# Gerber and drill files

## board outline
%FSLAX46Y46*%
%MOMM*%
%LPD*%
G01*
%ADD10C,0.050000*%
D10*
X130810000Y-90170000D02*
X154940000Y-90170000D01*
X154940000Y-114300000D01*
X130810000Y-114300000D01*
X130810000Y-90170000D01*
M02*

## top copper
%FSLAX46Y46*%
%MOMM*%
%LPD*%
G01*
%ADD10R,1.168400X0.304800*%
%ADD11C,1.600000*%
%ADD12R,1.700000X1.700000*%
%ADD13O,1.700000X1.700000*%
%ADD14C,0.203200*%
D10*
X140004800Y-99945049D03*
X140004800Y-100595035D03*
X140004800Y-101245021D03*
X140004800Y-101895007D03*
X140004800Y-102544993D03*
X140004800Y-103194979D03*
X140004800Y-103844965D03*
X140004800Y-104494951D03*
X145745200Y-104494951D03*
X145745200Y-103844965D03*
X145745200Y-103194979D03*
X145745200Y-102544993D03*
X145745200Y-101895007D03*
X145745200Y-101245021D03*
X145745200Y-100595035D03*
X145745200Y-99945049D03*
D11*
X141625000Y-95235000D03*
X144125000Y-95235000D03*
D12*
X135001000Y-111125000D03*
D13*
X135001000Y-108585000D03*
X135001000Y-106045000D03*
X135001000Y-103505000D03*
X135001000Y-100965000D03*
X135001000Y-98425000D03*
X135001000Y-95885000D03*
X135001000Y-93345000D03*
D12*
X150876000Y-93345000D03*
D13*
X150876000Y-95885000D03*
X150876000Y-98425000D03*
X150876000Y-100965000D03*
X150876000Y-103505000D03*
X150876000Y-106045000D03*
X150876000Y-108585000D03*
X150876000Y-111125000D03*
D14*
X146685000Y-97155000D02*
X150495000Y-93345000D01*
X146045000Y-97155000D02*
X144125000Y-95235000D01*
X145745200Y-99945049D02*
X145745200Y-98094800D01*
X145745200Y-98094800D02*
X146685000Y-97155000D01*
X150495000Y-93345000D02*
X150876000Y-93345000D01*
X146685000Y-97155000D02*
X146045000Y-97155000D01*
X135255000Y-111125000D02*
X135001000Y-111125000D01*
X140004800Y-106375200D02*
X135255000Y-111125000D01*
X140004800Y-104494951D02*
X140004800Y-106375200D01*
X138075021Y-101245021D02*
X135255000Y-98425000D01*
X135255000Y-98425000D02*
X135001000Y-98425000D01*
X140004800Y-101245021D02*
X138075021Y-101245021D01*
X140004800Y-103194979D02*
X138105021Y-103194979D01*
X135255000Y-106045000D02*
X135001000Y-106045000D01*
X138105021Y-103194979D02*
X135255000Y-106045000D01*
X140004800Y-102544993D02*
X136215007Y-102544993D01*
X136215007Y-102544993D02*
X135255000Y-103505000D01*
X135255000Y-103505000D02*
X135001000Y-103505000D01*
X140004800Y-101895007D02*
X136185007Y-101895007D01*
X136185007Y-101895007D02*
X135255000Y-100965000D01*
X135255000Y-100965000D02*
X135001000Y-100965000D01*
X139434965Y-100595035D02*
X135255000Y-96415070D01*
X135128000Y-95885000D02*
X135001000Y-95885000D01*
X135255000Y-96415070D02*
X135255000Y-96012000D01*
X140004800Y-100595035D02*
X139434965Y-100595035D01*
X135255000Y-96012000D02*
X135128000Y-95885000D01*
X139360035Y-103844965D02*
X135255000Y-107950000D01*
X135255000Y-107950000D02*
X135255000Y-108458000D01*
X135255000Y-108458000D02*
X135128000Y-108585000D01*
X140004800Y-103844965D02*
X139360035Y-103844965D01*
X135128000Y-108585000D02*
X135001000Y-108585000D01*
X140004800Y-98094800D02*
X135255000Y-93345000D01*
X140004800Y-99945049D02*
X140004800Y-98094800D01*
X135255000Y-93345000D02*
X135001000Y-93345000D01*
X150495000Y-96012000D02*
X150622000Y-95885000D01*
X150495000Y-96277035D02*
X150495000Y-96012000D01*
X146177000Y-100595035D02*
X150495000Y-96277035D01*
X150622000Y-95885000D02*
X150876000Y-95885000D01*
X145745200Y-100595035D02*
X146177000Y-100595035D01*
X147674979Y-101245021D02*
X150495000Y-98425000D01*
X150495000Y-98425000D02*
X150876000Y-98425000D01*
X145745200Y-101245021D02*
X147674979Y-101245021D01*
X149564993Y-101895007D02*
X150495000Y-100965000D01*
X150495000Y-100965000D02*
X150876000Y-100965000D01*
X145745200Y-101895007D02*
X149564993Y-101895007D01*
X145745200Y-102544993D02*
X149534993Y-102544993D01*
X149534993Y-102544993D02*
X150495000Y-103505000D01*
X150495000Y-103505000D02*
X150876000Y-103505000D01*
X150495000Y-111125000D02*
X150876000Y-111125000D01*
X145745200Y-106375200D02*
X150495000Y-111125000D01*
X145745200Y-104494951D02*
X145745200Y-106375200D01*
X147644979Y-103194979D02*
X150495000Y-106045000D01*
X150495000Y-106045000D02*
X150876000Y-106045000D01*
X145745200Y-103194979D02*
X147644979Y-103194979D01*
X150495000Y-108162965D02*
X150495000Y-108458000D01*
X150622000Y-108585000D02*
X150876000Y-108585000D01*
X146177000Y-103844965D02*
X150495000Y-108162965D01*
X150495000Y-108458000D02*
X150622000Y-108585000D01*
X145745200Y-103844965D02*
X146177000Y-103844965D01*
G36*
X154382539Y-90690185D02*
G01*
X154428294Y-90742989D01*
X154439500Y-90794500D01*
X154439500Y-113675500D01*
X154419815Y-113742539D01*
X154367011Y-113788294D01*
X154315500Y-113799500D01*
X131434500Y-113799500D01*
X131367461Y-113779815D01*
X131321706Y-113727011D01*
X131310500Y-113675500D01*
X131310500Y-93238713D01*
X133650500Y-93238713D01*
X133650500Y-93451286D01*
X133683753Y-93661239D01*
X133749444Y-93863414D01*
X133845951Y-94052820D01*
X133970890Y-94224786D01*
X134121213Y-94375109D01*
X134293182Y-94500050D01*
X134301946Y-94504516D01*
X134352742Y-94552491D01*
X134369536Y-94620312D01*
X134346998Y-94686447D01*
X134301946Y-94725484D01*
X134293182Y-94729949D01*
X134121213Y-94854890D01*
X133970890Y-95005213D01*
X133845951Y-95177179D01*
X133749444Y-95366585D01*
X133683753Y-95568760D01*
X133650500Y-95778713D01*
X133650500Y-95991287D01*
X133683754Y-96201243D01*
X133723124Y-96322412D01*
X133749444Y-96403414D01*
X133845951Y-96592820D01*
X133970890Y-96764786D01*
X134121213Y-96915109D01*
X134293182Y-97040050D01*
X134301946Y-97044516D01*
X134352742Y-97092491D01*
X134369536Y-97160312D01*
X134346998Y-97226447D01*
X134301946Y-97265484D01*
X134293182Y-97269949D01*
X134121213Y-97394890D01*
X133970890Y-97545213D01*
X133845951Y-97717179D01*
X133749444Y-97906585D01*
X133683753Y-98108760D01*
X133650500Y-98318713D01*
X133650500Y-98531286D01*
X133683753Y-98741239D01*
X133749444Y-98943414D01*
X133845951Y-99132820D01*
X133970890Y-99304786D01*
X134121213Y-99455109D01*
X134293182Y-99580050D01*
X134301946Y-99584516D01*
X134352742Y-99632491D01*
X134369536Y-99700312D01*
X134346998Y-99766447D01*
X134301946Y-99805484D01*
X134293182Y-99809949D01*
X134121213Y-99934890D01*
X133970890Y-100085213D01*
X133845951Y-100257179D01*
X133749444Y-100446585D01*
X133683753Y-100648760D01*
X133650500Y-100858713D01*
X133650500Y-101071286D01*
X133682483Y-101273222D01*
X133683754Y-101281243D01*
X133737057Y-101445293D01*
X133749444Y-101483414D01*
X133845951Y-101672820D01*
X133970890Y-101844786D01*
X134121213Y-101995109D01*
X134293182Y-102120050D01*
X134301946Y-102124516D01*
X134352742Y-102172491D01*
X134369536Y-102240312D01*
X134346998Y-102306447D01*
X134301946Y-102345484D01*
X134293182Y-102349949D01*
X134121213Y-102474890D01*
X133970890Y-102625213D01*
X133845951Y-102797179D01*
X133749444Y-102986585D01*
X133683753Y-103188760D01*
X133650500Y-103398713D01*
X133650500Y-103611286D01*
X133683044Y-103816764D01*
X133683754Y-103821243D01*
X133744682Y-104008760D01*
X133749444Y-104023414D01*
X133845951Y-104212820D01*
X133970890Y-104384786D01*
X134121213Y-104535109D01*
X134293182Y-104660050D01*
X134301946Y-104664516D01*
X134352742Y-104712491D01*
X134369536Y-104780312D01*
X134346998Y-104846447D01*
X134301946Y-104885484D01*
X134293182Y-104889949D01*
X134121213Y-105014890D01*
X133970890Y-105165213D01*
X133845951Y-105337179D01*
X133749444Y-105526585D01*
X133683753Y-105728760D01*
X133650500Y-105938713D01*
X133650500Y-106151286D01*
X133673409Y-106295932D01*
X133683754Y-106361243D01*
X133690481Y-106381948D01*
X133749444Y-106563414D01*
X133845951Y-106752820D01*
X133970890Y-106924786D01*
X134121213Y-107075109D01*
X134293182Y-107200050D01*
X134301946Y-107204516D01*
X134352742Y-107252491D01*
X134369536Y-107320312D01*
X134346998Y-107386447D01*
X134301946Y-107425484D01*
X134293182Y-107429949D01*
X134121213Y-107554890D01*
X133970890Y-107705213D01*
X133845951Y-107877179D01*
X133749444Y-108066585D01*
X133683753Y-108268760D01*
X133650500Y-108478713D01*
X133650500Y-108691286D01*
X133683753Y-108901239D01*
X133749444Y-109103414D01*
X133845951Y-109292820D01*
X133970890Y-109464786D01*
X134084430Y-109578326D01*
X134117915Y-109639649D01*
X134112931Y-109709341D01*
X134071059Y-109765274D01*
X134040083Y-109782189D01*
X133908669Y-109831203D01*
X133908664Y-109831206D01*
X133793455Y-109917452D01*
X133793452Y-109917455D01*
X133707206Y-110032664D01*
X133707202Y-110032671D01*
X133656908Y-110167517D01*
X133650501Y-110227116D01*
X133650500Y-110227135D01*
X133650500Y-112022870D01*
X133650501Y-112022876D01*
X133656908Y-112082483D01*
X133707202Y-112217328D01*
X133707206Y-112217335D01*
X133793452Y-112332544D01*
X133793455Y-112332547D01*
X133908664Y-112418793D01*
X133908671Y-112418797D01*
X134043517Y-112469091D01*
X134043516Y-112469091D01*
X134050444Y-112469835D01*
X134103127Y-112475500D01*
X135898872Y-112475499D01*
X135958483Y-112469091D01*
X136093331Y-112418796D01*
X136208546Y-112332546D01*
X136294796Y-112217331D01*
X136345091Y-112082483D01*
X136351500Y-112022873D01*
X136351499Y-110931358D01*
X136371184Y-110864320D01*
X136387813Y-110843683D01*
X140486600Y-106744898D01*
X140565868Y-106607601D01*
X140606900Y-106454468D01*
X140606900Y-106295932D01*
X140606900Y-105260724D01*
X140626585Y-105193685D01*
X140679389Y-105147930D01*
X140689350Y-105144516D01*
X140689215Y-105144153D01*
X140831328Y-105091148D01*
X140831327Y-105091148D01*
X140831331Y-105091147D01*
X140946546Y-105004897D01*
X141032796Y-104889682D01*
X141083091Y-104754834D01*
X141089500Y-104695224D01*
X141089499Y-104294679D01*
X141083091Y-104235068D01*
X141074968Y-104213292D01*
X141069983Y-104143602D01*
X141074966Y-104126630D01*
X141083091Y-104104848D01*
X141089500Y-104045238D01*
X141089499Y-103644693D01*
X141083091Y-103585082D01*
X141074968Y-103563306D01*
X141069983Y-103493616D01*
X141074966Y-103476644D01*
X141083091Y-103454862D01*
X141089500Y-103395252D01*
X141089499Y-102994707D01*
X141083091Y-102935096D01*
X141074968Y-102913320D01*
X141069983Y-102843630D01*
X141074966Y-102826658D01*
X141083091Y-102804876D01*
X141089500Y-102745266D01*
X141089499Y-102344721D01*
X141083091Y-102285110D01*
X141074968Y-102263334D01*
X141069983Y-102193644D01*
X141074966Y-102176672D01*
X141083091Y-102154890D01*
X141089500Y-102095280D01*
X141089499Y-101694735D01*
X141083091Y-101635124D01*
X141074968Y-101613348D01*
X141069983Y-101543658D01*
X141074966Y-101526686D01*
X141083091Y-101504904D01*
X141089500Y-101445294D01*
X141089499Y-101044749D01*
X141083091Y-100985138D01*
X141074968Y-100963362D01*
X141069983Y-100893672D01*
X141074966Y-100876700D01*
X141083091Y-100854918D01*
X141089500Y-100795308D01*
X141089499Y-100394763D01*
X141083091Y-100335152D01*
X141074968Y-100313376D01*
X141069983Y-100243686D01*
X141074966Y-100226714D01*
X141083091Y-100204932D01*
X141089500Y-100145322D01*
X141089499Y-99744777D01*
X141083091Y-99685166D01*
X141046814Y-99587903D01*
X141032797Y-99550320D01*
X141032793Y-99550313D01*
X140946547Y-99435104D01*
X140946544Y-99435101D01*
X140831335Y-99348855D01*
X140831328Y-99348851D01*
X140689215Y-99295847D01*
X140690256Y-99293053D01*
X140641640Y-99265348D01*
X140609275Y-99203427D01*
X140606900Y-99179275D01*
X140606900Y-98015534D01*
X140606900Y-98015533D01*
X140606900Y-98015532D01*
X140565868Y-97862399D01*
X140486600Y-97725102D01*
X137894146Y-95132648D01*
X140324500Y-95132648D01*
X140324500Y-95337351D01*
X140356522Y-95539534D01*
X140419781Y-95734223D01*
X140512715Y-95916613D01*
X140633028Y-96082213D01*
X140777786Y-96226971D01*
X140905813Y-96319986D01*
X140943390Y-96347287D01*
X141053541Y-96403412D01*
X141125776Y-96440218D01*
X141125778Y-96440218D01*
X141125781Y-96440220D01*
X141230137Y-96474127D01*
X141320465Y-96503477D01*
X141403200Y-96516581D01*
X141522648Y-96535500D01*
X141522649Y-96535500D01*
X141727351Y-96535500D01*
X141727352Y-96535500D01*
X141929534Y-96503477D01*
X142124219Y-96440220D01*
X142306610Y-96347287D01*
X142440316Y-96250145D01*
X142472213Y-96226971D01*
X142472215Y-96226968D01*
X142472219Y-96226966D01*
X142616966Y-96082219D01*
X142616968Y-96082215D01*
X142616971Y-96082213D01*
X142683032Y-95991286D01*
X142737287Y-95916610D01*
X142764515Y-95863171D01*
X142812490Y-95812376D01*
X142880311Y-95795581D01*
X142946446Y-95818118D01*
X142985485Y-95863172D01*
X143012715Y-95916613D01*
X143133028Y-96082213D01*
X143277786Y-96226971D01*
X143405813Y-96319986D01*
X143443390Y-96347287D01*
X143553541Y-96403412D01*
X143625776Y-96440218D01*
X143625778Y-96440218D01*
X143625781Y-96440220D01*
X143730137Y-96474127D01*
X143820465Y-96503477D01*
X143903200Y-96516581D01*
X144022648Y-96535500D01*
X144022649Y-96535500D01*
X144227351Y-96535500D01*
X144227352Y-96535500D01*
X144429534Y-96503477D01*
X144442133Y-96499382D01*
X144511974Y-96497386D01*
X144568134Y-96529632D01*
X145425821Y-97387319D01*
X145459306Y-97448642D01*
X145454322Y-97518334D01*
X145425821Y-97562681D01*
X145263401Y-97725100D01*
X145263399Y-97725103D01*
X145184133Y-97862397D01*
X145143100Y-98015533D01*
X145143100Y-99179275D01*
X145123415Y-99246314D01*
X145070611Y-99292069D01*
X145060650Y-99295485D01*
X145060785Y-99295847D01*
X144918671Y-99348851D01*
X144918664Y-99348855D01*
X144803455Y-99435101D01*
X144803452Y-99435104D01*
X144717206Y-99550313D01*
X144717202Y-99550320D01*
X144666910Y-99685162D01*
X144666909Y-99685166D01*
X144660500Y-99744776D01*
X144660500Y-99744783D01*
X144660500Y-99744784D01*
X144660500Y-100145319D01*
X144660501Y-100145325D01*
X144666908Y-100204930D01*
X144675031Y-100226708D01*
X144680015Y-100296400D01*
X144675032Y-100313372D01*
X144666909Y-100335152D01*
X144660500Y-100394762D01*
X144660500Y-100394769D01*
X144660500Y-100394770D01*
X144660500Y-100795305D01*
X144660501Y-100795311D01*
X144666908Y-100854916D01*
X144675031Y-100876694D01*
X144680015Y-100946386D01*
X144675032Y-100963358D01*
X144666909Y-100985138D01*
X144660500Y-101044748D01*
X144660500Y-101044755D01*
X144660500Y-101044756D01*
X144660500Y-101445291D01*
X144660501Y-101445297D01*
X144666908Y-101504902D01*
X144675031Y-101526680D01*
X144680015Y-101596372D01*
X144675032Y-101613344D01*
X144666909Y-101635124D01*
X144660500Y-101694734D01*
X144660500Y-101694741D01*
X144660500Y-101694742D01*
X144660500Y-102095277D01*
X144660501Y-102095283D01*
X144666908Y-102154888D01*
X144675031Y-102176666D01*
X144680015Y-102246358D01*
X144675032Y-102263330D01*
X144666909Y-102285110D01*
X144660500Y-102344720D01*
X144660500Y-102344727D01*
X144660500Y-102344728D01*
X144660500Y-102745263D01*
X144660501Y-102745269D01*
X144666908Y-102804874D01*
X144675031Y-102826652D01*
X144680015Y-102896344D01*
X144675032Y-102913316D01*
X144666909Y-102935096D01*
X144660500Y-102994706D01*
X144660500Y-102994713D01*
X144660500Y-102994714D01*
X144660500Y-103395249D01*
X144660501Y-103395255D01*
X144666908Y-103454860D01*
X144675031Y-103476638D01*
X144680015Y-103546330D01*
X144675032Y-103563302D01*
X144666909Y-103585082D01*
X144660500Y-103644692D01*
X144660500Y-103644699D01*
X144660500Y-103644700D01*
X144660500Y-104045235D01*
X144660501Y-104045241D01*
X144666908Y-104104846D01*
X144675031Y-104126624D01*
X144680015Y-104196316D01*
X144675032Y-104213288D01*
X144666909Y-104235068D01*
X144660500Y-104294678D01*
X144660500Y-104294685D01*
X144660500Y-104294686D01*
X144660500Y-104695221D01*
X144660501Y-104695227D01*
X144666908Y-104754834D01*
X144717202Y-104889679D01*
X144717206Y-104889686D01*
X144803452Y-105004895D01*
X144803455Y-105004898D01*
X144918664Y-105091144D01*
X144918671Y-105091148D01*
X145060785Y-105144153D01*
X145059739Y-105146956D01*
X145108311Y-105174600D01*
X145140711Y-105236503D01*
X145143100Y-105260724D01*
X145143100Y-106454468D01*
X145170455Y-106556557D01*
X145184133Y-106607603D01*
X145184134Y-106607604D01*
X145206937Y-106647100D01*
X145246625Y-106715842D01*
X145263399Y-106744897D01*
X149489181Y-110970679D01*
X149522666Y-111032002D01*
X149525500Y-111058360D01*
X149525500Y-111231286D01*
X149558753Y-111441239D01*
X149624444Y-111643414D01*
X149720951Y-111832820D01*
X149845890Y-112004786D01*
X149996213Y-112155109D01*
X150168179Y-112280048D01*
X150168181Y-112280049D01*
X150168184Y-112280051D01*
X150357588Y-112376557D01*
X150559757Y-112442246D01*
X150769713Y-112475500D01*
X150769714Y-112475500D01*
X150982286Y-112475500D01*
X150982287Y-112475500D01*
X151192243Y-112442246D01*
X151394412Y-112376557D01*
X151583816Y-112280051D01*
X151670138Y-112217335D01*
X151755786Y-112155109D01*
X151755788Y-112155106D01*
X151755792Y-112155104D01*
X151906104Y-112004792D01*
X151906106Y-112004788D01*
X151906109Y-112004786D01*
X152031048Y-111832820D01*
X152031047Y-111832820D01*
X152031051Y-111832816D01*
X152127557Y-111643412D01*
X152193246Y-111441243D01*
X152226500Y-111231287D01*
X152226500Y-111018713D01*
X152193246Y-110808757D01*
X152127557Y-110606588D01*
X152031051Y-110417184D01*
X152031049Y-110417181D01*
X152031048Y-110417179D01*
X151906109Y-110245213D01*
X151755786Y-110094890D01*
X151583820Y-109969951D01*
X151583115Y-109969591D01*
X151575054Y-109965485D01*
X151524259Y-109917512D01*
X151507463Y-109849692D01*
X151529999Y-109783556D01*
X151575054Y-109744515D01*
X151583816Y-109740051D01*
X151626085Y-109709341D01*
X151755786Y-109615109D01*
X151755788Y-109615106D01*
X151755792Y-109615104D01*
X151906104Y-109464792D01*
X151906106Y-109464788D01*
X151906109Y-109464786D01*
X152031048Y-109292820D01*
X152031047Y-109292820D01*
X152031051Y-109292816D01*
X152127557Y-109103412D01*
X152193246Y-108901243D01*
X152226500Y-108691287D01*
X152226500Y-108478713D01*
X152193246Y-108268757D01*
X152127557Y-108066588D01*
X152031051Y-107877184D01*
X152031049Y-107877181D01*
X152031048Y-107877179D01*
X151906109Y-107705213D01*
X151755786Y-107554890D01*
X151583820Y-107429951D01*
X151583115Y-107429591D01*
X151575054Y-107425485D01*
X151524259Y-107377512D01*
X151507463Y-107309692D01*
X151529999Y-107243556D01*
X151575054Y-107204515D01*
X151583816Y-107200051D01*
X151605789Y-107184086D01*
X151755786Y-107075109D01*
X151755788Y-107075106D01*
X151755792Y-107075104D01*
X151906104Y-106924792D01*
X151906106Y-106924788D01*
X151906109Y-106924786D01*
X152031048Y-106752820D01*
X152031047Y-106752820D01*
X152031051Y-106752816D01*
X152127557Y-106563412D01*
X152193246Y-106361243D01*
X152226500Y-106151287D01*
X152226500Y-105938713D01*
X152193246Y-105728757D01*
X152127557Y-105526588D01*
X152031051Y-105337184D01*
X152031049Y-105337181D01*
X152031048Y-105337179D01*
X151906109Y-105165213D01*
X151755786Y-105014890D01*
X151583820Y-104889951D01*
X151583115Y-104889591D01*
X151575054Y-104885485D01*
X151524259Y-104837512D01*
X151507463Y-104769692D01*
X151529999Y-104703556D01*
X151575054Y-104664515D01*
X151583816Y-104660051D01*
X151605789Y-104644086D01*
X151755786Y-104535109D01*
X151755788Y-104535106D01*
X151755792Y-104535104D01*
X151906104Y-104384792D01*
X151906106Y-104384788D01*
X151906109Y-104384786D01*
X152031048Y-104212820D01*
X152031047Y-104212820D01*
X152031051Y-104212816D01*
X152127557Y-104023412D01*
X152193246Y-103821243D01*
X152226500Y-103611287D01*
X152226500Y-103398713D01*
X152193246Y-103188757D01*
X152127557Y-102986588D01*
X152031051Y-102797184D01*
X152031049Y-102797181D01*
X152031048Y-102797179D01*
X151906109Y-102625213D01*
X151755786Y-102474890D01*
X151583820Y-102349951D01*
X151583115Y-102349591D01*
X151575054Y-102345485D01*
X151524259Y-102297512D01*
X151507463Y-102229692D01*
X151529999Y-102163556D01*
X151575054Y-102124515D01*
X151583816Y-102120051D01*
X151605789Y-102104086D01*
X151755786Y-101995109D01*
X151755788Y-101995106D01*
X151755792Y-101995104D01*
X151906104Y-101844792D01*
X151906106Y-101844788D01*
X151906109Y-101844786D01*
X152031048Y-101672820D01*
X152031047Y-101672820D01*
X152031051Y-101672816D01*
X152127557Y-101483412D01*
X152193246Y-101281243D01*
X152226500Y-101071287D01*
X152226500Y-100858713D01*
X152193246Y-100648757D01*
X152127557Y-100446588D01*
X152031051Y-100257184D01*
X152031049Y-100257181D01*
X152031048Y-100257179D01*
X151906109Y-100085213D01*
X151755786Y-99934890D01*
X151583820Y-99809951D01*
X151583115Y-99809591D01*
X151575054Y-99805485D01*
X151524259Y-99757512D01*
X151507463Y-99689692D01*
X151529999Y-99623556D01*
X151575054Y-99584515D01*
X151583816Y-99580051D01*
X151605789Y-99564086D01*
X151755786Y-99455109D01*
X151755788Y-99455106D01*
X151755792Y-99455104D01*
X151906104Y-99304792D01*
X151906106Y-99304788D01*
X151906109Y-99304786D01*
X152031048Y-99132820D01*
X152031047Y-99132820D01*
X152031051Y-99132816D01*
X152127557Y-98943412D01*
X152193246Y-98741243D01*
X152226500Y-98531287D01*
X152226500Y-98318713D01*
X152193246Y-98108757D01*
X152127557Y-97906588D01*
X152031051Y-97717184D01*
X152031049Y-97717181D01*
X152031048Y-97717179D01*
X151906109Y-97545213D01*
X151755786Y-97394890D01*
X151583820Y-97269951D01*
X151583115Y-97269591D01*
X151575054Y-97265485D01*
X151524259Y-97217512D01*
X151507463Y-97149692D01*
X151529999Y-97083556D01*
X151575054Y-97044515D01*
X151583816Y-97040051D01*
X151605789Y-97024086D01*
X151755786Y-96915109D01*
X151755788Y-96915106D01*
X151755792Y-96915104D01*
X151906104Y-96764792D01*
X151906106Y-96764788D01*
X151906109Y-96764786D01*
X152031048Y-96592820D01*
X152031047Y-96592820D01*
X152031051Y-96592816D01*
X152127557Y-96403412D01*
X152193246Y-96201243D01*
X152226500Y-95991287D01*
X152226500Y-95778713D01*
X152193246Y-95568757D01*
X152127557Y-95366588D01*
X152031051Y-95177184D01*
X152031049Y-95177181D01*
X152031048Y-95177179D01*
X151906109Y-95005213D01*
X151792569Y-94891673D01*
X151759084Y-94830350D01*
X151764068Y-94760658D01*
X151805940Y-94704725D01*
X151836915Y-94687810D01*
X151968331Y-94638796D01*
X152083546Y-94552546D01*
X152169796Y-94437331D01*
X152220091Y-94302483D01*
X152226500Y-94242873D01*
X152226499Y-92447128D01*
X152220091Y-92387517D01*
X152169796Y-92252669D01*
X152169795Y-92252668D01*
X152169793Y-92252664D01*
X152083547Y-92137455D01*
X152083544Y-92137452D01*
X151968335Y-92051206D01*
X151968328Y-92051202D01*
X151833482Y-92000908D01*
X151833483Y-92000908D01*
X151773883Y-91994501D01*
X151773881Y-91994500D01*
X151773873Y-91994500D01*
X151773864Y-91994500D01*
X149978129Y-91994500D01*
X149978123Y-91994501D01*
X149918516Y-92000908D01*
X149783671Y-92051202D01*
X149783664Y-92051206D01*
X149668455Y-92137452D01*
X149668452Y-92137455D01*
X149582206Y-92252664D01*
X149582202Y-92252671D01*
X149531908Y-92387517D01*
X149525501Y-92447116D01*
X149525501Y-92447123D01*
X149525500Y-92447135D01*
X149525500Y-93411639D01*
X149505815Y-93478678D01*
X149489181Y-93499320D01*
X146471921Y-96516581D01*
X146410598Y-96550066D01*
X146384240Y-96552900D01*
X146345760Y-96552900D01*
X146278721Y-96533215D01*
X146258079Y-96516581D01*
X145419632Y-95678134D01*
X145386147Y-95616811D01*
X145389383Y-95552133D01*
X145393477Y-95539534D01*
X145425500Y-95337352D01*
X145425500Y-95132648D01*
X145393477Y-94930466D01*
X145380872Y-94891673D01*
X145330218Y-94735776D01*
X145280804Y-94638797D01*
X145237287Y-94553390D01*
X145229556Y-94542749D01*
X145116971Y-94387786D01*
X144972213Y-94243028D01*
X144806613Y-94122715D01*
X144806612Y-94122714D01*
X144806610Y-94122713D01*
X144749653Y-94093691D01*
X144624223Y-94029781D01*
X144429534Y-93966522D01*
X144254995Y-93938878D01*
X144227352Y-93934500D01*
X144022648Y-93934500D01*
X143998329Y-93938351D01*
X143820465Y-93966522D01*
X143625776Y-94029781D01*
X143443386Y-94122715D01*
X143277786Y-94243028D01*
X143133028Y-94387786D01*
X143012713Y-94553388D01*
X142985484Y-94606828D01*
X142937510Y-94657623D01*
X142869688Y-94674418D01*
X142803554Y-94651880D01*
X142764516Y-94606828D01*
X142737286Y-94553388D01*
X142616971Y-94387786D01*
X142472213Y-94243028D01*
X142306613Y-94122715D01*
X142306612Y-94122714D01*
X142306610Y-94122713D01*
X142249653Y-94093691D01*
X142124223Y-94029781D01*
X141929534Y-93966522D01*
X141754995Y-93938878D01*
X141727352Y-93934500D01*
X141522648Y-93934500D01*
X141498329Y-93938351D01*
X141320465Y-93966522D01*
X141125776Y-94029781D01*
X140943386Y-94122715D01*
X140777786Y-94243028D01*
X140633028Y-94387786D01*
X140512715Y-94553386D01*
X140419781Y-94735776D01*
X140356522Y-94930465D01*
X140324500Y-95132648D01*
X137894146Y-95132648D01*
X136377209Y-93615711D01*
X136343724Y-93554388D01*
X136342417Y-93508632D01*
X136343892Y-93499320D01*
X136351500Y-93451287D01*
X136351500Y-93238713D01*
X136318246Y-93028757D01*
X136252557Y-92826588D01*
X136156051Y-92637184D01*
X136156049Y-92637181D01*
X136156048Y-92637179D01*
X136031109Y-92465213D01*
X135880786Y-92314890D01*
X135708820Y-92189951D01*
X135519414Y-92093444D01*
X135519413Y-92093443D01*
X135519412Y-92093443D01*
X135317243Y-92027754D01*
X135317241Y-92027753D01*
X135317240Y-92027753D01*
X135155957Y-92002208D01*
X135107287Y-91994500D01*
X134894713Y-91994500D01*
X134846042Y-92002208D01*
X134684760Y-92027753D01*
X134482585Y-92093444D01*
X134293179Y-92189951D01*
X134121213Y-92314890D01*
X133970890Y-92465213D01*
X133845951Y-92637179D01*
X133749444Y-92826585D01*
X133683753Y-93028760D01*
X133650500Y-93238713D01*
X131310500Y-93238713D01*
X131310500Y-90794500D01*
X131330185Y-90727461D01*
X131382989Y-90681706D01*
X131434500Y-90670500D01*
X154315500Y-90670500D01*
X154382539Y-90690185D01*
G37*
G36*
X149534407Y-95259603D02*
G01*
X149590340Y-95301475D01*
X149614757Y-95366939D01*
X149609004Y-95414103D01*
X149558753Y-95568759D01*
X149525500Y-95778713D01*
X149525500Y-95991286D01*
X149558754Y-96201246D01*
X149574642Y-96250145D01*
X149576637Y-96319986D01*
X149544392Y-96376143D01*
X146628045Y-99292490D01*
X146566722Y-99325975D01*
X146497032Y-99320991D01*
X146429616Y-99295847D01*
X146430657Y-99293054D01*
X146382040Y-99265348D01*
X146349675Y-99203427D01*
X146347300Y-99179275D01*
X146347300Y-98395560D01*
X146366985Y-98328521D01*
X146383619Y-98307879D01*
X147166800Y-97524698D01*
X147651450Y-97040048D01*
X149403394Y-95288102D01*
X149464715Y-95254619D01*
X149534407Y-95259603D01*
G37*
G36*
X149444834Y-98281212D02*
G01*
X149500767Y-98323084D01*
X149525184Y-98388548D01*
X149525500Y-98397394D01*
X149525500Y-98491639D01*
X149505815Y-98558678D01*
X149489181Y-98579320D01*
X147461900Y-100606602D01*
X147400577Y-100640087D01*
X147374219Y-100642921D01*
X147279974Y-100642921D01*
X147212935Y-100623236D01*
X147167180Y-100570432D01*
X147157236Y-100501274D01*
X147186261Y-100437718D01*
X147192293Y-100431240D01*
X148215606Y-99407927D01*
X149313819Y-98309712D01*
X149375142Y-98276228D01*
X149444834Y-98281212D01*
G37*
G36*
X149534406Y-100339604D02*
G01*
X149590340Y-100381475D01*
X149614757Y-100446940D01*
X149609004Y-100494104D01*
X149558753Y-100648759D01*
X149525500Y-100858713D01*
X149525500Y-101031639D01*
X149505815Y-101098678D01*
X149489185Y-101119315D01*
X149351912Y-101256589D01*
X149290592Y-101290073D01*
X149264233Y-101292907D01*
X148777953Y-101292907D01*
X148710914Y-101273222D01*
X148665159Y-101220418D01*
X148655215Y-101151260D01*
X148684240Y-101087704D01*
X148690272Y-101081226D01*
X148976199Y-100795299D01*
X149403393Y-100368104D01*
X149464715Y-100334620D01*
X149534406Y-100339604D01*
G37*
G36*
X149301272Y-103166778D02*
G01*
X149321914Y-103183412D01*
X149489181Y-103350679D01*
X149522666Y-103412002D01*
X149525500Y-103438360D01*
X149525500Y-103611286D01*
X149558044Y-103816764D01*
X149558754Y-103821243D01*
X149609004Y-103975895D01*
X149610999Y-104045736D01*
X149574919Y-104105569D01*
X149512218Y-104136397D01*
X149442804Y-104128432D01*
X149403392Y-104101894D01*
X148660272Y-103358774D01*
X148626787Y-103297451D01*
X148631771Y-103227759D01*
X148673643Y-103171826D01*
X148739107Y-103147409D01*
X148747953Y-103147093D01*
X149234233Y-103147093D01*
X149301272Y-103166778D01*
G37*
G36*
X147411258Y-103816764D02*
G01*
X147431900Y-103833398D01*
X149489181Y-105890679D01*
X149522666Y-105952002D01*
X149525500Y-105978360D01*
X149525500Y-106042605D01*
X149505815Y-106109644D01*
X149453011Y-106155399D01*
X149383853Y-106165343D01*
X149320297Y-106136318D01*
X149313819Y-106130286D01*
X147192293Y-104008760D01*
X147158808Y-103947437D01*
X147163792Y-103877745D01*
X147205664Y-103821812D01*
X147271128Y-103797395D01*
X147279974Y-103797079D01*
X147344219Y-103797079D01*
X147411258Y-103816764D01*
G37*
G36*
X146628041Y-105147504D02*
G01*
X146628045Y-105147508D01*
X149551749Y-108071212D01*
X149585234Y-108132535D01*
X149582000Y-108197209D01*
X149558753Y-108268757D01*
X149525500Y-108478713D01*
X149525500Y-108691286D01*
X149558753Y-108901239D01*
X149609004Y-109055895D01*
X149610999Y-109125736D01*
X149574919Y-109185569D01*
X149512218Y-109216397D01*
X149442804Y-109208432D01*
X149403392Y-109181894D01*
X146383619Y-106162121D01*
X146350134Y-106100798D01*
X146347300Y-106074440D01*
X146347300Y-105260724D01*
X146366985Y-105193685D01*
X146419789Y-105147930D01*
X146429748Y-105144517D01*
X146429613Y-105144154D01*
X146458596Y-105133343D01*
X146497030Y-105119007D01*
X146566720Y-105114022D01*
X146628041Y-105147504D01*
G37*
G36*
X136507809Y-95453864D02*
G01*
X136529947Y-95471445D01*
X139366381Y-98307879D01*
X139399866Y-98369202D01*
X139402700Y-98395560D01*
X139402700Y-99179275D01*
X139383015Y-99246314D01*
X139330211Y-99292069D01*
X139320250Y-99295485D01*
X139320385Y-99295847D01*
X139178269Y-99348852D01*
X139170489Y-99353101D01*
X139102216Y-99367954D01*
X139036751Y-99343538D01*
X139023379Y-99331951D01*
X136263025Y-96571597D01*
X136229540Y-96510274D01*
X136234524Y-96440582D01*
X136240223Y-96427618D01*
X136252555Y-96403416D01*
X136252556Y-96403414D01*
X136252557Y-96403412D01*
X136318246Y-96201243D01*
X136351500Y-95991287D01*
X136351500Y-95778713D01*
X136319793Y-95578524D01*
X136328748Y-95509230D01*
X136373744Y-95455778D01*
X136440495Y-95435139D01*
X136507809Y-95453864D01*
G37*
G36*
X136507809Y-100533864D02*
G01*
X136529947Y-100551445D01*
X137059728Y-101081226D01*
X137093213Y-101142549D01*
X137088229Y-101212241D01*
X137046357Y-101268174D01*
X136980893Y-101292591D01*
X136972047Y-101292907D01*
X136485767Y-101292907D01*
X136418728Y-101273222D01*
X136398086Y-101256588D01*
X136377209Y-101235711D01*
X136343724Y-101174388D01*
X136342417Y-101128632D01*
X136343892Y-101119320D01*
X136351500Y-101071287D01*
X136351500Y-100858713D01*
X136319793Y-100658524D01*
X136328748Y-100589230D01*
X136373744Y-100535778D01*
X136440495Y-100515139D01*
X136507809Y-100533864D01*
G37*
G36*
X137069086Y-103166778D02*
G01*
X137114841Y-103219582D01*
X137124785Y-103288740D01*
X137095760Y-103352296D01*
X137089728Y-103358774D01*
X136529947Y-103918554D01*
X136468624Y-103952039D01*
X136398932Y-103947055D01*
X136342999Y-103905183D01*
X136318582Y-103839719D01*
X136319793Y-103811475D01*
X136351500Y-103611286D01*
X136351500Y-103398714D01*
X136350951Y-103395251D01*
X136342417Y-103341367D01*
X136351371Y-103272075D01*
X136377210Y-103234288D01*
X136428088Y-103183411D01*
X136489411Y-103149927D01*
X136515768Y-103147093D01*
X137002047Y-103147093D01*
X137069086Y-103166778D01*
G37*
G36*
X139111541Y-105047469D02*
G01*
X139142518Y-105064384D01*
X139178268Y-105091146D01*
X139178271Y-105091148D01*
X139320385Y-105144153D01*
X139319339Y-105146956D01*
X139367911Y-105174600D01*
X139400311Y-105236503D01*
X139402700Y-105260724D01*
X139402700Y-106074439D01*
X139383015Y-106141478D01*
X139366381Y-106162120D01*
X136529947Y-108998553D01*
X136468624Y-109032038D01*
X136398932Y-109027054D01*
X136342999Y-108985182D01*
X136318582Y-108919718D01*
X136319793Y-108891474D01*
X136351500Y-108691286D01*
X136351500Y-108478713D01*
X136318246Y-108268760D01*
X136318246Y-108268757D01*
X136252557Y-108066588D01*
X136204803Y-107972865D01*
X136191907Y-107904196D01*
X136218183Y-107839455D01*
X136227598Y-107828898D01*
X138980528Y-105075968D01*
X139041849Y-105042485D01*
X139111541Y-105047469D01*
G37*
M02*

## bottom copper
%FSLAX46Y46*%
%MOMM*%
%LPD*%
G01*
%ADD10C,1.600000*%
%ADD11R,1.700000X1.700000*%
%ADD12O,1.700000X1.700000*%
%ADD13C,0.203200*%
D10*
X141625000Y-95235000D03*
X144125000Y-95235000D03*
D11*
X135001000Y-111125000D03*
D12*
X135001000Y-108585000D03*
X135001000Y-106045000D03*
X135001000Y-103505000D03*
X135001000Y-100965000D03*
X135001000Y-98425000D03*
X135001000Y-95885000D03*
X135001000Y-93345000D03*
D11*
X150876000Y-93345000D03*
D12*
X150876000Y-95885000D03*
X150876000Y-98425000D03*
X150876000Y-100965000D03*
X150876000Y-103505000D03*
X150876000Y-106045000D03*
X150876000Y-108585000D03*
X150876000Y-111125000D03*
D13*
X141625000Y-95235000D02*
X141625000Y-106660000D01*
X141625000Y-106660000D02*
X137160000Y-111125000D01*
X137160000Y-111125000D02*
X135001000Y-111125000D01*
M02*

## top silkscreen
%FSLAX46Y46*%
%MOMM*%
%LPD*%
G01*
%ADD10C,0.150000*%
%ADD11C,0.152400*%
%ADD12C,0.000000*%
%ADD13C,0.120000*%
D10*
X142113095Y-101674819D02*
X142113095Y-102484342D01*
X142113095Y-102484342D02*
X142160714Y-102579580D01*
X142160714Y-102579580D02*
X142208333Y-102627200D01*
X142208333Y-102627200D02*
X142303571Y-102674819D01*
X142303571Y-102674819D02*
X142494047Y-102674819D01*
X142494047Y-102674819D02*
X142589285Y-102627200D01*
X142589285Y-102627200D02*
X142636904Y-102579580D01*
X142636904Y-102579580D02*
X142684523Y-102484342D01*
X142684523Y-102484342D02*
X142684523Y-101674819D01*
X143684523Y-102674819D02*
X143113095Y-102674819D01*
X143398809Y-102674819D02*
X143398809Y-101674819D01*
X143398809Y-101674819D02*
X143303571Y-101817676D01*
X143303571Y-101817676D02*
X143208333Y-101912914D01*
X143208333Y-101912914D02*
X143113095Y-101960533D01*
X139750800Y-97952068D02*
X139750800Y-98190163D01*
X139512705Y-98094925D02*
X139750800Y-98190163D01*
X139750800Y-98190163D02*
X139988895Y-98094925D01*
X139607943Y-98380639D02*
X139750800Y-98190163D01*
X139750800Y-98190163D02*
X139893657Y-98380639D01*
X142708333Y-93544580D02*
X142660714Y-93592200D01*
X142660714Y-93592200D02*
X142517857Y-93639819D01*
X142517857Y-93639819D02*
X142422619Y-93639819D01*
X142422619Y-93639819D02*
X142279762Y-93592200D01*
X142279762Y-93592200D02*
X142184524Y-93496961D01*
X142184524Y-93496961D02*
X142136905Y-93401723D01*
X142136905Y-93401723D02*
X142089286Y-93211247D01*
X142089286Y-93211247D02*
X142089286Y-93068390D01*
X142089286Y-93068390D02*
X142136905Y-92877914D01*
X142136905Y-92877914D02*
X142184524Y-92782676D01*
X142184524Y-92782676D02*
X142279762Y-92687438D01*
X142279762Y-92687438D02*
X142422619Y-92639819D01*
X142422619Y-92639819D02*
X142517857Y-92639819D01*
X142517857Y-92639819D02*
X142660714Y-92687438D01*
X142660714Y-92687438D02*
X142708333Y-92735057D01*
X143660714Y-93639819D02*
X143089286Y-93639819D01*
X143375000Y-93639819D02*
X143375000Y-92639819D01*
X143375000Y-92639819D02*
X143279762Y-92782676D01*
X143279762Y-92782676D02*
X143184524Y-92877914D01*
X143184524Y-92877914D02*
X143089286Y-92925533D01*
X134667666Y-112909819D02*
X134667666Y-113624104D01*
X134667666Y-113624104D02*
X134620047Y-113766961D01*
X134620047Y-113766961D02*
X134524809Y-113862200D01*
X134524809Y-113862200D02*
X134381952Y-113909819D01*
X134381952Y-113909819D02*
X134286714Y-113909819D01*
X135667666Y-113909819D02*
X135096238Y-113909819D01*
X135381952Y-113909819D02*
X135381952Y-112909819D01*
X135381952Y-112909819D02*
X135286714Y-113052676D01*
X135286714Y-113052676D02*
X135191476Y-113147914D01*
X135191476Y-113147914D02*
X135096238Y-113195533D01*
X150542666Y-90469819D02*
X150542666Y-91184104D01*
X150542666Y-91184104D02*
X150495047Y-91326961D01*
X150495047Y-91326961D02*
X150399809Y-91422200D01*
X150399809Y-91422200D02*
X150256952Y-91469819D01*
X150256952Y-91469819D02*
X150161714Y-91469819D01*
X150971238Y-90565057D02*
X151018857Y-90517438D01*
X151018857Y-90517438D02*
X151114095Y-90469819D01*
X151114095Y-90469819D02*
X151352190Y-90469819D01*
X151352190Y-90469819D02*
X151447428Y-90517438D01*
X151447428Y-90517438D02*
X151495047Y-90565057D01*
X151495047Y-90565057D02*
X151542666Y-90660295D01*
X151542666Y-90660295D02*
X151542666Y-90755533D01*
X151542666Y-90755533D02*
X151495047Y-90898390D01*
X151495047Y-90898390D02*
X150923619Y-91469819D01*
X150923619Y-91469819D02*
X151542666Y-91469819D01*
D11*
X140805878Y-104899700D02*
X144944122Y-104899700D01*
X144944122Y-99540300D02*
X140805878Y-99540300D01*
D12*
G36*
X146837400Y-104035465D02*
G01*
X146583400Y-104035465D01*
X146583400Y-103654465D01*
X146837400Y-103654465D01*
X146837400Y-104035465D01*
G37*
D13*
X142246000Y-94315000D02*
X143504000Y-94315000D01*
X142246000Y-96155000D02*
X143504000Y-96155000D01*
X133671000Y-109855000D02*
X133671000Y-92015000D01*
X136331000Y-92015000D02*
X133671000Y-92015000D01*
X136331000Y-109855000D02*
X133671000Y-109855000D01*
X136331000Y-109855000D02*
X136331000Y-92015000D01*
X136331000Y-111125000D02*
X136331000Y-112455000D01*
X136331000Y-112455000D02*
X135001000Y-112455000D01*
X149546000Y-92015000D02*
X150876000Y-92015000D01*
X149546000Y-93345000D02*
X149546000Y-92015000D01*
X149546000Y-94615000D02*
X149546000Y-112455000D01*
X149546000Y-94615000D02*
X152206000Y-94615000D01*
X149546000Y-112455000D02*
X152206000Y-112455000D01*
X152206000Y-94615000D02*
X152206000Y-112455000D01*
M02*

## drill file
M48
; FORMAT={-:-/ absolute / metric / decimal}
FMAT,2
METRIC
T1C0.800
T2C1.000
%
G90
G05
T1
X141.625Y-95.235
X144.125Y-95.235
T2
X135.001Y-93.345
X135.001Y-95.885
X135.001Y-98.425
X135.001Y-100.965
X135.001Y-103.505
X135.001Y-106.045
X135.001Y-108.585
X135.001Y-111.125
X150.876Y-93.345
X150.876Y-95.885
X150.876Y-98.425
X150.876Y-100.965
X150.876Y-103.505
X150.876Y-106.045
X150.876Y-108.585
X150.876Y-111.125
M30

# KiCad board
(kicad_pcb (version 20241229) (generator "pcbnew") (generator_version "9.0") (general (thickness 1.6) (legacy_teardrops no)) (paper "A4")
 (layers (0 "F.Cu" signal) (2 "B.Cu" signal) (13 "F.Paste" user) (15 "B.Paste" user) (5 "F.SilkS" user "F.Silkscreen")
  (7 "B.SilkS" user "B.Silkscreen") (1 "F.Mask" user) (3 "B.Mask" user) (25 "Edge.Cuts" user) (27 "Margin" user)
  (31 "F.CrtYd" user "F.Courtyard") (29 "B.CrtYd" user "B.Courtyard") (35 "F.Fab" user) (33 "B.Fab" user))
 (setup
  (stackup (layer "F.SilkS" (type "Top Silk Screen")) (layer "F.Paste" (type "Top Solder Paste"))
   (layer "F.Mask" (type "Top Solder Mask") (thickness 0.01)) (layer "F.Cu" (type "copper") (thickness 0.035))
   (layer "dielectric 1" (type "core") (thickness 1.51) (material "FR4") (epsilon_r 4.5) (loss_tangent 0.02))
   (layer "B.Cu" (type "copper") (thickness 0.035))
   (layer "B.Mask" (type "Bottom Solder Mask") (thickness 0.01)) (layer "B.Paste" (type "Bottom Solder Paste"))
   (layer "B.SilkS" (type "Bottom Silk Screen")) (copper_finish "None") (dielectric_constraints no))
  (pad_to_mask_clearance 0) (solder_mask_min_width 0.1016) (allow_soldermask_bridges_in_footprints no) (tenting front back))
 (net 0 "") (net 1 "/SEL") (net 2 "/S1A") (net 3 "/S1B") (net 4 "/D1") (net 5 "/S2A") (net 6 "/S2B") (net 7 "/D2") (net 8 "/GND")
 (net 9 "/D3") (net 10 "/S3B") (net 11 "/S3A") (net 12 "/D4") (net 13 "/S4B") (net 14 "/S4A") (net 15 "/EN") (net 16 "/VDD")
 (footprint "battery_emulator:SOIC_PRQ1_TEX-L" (layer "F.Cu") (at 142.875 102.22)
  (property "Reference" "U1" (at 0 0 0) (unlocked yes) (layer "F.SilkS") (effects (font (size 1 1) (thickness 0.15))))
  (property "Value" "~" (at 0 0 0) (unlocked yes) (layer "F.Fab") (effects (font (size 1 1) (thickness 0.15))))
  (fp_line (start -2.069122 2.6797) (end 2.069122 2.6797) (stroke (width 0.1524) (type solid)) (layer "F.SilkS"))
  (fp_line (start 2.069122 -2.6797) (end -2.069122 -2.6797) (stroke (width 0.1524) (type solid)) (layer "F.SilkS"))
  (fp_poly
   (pts (xy 3.9624 1.434465) (xy 3.9624 1.815465) (xy 3.7084 1.815465) (xy 3.7084 1.434465)) (stroke (width 0) (type solid)) (fill yes)
   (layer "F.SilkS"))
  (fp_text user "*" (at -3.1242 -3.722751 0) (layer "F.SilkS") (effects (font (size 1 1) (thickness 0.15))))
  (pad "1" smd rect (at -2.8702 -2.274951) (size 1.1684 0.3048) (layers "F.Cu" "F.Mask" "F.Paste") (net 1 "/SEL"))
  (pad "2" smd rect (at -2.8702 -1.624965) (size 1.1684 0.3048) (layers "F.Cu" "F.Mask" "F.Paste") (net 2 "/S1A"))
  (pad "3" smd rect (at -2.8702 -0.974979) (size 1.1684 0.3048) (layers "F.Cu" "F.Mask" "F.Paste") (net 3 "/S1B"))
  (pad "4" smd rect (at -2.8702 -0.324993) (size 1.1684 0.3048) (layers "F.Cu" "F.Mask" "F.Paste") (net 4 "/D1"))
  (pad "5" smd rect (at -2.8702 0.324993) (size 1.1684 0.3048) (layers "F.Cu" "F.Mask" "F.Paste") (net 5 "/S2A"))
  (pad "6" smd rect (at -2.8702 0.974979) (size 1.1684 0.3048) (layers "F.Cu" "F.Mask" "F.Paste") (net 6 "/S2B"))
  (pad "7" smd rect (at -2.8702 1.624965) (size 1.1684 0.3048) (layers "F.Cu" "F.Mask" "F.Paste") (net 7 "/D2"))
  (pad "8" smd rect (at -2.8702 2.274951) (size 1.1684 0.3048) (layers "F.Cu" "F.Mask" "F.Paste") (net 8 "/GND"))
  (pad "9" smd rect (at 2.8702 2.274951) (size 1.1684 0.3048) (layers "F.Cu" "F.Mask" "F.Paste") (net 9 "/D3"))
  (pad "10" smd rect (at 2.8702 1.624965) (size 1.1684 0.3048) (layers "F.Cu" "F.Mask" "F.Paste") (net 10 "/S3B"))
  (pad "11" smd rect (at 2.8702 0.974979) (size 1.1684 0.3048) (layers "F.Cu" "F.Mask" "F.Paste") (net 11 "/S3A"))
  (pad "12" smd rect (at 2.8702 0.324993) (size 1.1684 0.3048) (layers "F.Cu" "F.Mask" "F.Paste") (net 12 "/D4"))
  (pad "13" smd rect (at 2.8702 -0.324993) (size 1.1684 0.3048) (layers "F.Cu" "F.Mask" "F.Paste") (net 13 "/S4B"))
  (pad "14" smd rect (at 2.8702 -0.974979) (size 1.1684 0.3048) (layers "F.Cu" "F.Mask" "F.Paste") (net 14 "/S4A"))
  (pad "15" smd rect (at 2.8702 -1.624965) (size 1.1684 0.3048) (layers "F.Cu" "F.Mask" "F.Paste") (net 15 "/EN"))
  (pad "16" smd rect (at 2.8702 -2.274951) (size 1.1684 0.3048) (layers "F.Cu" "F.Mask" "F.Paste") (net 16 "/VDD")))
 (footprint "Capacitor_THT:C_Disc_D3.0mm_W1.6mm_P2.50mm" (layer "F.Cu") (at 141.625 95.235)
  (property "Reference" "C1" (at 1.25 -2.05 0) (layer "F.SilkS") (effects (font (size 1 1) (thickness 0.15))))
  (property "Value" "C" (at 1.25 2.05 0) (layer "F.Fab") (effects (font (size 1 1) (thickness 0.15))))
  (fp_line (start 0.621 -0.92) (end 1.879 -0.92) (stroke (width 0.12) (type solid)) (layer "F.SilkS"))
  (fp_line (start 0.621 0.92) (end 1.879 0.92) (stroke (width 0.12) (type solid)) (layer "F.SilkS"))
  (pad "1" thru_hole circle (at 0 0) (size 1.6 1.6) (drill 0.8) (layers "*.Cu" "*.Mask") (remove_unused_layers no) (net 8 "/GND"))
  (pad "2" thru_hole circle (at 2.5 0) (size 1.6 1.6) (drill 0.8) (layers "*.Cu" "*.Mask") (remove_unused_layers no) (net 16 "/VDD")))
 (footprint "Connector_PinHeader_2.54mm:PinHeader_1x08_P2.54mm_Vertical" (layer "F.Cu") (at 135.001 111.125 180)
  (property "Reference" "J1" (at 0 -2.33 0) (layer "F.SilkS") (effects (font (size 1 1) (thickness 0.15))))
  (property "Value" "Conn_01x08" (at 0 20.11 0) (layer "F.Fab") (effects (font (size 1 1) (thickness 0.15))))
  (fp_line (start 1.33 1.27) (end 1.33 19.11) (stroke (width 0.12) (type solid)) (layer "F.SilkS"))
  (fp_line (start -1.33 19.11) (end 1.33 19.11) (stroke (width 0.12) (type solid)) (layer "F.SilkS"))
  (fp_line (start -1.33 1.27) (end 1.33 1.27) (stroke (width 0.12) (type solid)) (layer "F.SilkS"))
  (fp_line (start -1.33 1.27) (end -1.33 19.11) (stroke (width 0.12) (type solid)) (layer "F.SilkS"))
  (fp_line (start -1.33 0) (end -1.33 -1.33) (stroke (width 0.12) (type solid)) (layer "F.SilkS"))
  (fp_line (start -1.33 -1.33) (end 0 -1.33) (stroke (width 0.12) (type solid)) (layer "F.SilkS"))
  (pad "1" thru_hole rect (at 0 0 180) (size 1.7 1.7) (drill 1) (layers "*.Cu" "*.Mask") (remove_unused_layers no) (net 8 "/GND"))
  (pad "2" thru_hole oval (at 0 2.54 180) (size 1.7 1.7) (drill 1) (layers "*.Cu" "*.Mask") (remove_unused_layers no) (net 7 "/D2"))
  (pad "3" thru_hole oval (at 0 5.08 180) (size 1.7 1.7) (drill 1) (layers "*.Cu" "*.Mask") (remove_unused_layers no) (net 6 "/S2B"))
  (pad "4" thru_hole oval (at 0 7.62 180) (size 1.7 1.7) (drill 1) (layers "*.Cu" "*.Mask") (remove_unused_layers no) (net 5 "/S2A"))
  (pad "5" thru_hole oval (at 0 10.16 180) (size 1.7 1.7) (drill 1) (layers "*.Cu" "*.Mask") (remove_unused_layers no) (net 4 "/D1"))
  (pad "6" thru_hole oval (at 0 12.7 180) (size 1.7 1.7) (drill 1) (layers "*.Cu" "*.Mask") (remove_unused_layers no) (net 3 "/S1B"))
  (pad "7" thru_hole oval (at 0 15.24 180) (size 1.7 1.7) (drill 1) (layers "*.Cu" "*.Mask") (remove_unused_layers no) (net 2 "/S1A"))
  (pad "8" thru_hole oval (at 0 17.78 180) (size 1.7 1.7) (drill 1) (layers "*.Cu" "*.Mask") (remove_unused_layers no) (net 1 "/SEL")))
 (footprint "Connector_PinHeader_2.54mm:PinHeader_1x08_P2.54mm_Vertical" (layer "F.Cu") (at 150.876 93.345)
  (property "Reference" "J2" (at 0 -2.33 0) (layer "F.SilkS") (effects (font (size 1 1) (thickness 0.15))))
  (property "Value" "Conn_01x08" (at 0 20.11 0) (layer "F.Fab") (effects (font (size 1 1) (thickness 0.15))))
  (fp_line (start -1.33 -1.33) (end 0 -1.33) (stroke (width 0.12) (type solid)) (layer "F.SilkS"))
  (fp_line (start -1.33 0) (end -1.33 -1.33) (stroke (width 0.12) (type solid)) (layer "F.SilkS"))
  (fp_line (start -1.33 1.27) (end -1.33 19.11) (stroke (width 0.12) (type solid)) (layer "F.SilkS"))
  (fp_line (start -1.33 1.27) (end 1.33 1.27) (stroke (width 0.12) (type solid)) (layer "F.SilkS"))
  (fp_line (start -1.33 19.11) (end 1.33 19.11) (stroke (width 0.12) (type solid)) (layer "F.SilkS"))
  (fp_line (start 1.33 1.27) (end 1.33 19.11) (stroke (width 0.12) (type solid)) (layer "F.SilkS"))
  (pad "1" thru_hole rect (at 0 0) (size 1.7 1.7) (drill 1) (layers "*.Cu" "*.Mask") (remove_unused_layers no) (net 16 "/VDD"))
  (pad "2" thru_hole oval (at 0 2.54) (size 1.7 1.7) (drill 1) (layers "*.Cu" "*.Mask") (remove_unused_layers no) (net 15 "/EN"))
  (pad "3" thru_hole oval (at 0 5.08) (size 1.7 1.7) (drill 1) (layers "*.Cu" "*.Mask") (remove_unused_layers no) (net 14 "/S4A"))
  (pad "4" thru_hole oval (at 0 7.62) (size 1.7 1.7) (drill 1) (layers "*.Cu" "*.Mask") (remove_unused_layers no) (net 13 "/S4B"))
  (pad "5" thru_hole oval (at 0 10.16) (size 1.7 1.7) (drill 1) (layers "*.Cu" "*.Mask") (remove_unused_layers no) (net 12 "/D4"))
  (pad "6" thru_hole oval (at 0 12.7) (size 1.7 1.7) (drill 1) (layers "*.Cu" "*.Mask") (remove_unused_layers no) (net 11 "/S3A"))
  (pad "7" thru_hole oval (at 0 15.24) (size 1.7 1.7) (drill 1) (layers "*.Cu" "*.Mask") (remove_unused_layers no) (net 10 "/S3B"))
  (pad "8" thru_hole oval (at 0 17.78) (size 1.7 1.7) (drill 1) (layers "*.Cu" "*.Mask") (remove_unused_layers no) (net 9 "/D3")))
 (gr_rect (start 130.81 90.17) (end 154.94 114.3) (stroke (width 0.05) (type solid)) (fill no) (layer "Edge.Cuts"))
 (segment (start 146.685 97.155) (end 150.495 93.345) (width 0.2032) (layer "F.Cu") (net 16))
 (segment (start 146.045 97.155) (end 144.125 95.235) (width 0.2032) (layer "F.Cu") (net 16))
 (segment (start 145.7452 99.945049) (end 145.7452 98.0948) (width 0.2032) (layer "F.Cu") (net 16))
 (segment (start 145.7452 98.0948) (end 146.685 97.155) (width 0.2032) (layer "F.Cu") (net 16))
 (segment (start 150.495 93.345) (end 150.876 93.345) (width 0.2032) (layer "F.Cu") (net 16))
 (segment (start 146.685 97.155) (end 146.045 97.155) (width 0.2032) (layer "F.Cu") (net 16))
 (segment (start 135.255 111.125) (end 135.001 111.125) (width 0.2032) (layer "F.Cu") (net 8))
 (segment (start 140.0048 106.3752) (end 135.255 111.125) (width 0.2032) (layer "F.Cu") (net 8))
 (segment (start 140.0048 104.494951) (end 140.0048 106.3752) (width 0.2032) (layer "F.Cu") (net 8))
 (segment (start 141.625 95.235) (end 141.625 106.66) (width 0.2032) (layer "B.Cu") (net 8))
 (segment (start 141.625 106.66) (end 137.16 111.125) (width 0.2032) (layer "B.Cu") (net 8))
 (segment (start 137.16 111.125) (end 135.001 111.125) (width 0.2032) (layer "B.Cu") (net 8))
 (segment (start 138.075021 101.245021) (end 135.255 98.425) (width 0.2032) (layer "F.Cu") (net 3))
 (segment (start 135.255 98.425) (end 135.001 98.425) (width 0.2032) (layer "F.Cu") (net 3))
 (segment (start 140.0048 101.245021) (end 138.075021 101.245021) (width 0.2032) (layer "F.Cu") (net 3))
 (segment (start 140.0048 103.194979) (end 138.105021 103.194979) (width 0.2032) (layer "F.Cu") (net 6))
 (segment (start 135.255 106.045) (end 135.001 106.045) (width 0.2032) (layer "F.Cu") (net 6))
 (segment (start 138.105021 103.194979) (end 135.255 106.045) (width 0.2032) (layer "F.Cu") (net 6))
 (segment (start 140.0048 102.544993) (end 136.215007 102.544993) (width 0.2032) (layer "F.Cu") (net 5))
 (segment (start 136.215007 102.544993) (end 135.255 103.505) (width 0.2032) (layer "F.Cu") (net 5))
 (segment (start 135.255 103.505) (end 135.001 103.505) (width 0.2032) (layer "F.Cu") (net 5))
 (segment (start 140.0048 101.895007) (end 136.185007 101.895007) (width 0.2032) (layer "F.Cu") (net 4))
 (segment (start 136.185007 101.895007) (end 135.255 100.965) (width 0.2032) (layer "F.Cu") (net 4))
 (segment (start 135.255 100.965) (end 135.001 100.965) (width 0.2032) (layer "F.Cu") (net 4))
 (segment (start 139.434965 100.595035) (end 135.255 96.41507) (width 0.2032) (layer "F.Cu") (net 2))
 (segment (start 135.128 95.885) (end 135.001 95.885) (width 0.2032) (layer "F.Cu") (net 2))
 (segment (start 135.255 96.41507) (end 135.255 96.012) (width 0.2032) (layer "F.Cu") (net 2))
 (segment (start 140.0048 100.595035) (end 139.434965 100.595035) (width 0.2032) (layer "F.Cu") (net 2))
 (segment (start 135.255 96.012) (end 135.128 95.885) (width 0.2032) (layer "F.Cu") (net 2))
 (segment (start 139.360035 103.844965) (end 135.255 107.95) (width 0.2032) (layer "F.Cu") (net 7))
 (segment (start 135.255 107.95) (end 135.255 108.458) (width 0.2032) (layer "F.Cu") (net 7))
 (segment (start 135.255 108.458) (end 135.128 108.585) (width 0.2032) (layer "F.Cu") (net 7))
 (segment (start 140.0048 103.844965) (end 139.360035 103.844965) (width 0.2032) (layer "F.Cu") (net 7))
 (segment (start 135.128 108.585) (end 135.001 108.585) (width 0.2032) (layer "F.Cu") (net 7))
 (segment (start 140.0048 98.0948) (end 135.255 93.345) (width 0.2032) (layer "F.Cu") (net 1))
 (segment (start 140.0048 99.945049) (end 140.0048 98.0948) (width 0.2032) (layer "F.Cu") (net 1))
 (segment (start 135.255 93.345) (end 135.001 93.345) (width 0.2032) (layer "F.Cu") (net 1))
 (segment (start 150.495 96.012) (end 150.622 95.885) (width 0.2032) (layer "F.Cu") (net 15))
 (segment (start 150.495 96.277035) (end 150.495 96.012) (width 0.2032) (layer "F.Cu") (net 15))
 (segment (start 146.177 100.595035) (end 150.495 96.277035) (width 0.2032) (layer "F.Cu") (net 15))
 (segment (start 150.622 95.885) (end 150.876 95.885) (width 0.2032) (layer "F.Cu") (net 15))
 (segment (start 145.7452 100.595035) (end 146.177 100.595035) (width 0.2032) (layer "F.Cu") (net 15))
 (segment (start 147.674979 101.245021) (end 150.495 98.425) (width 0.2032) (layer "F.Cu") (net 14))
 (segment (start 150.495 98.425) (end 150.876 98.425) (width 0.2032) (layer "F.Cu") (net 14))
 (segment (start 145.7452 101.245021) (end 147.674979 101.245021) (width 0.2032) (layer "F.Cu") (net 14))
 (segment (start 149.564993 101.895007) (end 150.495 100.965) (width 0.2032) (layer "F.Cu") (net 13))
 (segment (start 150.495 100.965) (end 150.876 100.965) (width 0.2032) (layer "F.Cu") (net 13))
 (segment (start 145.7452 101.895007) (end 149.564993 101.895007) (width 0.2032) (layer "F.Cu") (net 13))
 (segment (start 145.7452 102.544993) (end 149.534993 102.544993) (width 0.2032) (layer "F.Cu") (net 12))
 (segment (start 149.534993 102.544993) (end 150.495 103.505) (width 0.2032) (layer "F.Cu") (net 12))
 (segment (start 150.495 103.505) (end 150.876 103.505) (width 0.2032) (layer "F.Cu") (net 12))
 (segment (start 150.495 111.125) (end 150.876 111.125) (width 0.2032) (layer "F.Cu") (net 9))
 (segment (start 145.7452 106.3752) (end 150.495 111.125) (width 0.2032) (layer "F.Cu") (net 9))
 (segment (start 145.7452 104.494951) (end 145.7452 106.3752) (width 0.2032) (layer "F.Cu") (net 9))
 (segment (start 147.644979 103.194979) (end 150.495 106.045) (width 0.2032) (layer "F.Cu") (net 11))
 (segment (start 150.495 106.045) (end 150.876 106.045) (width 0.2032) (layer "F.Cu") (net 11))
 (segment (start 145.7452 103.194979) (end 147.644979 103.194979) (width 0.2032) (layer "F.Cu") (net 11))
 (segment (start 150.495 108.162965) (end 150.495 108.458) (width 0.2032) (layer "F.Cu") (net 10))
 (segment (start 150.622 108.585) (end 150.876 108.585) (width 0.2032) (layer "F.Cu") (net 10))
 (segment (start 146.177 103.844965) (end 150.495 108.162965) (width 0.2032) (layer "F.Cu") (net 10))
 (segment (start 150.495 108.458) (end 150.622 108.585) (width 0.2032) (layer "F.Cu") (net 10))
 (segment (start 145.7452 103.844965) (end 146.177 103.844965) (width 0.2032) (layer "F.Cu") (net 10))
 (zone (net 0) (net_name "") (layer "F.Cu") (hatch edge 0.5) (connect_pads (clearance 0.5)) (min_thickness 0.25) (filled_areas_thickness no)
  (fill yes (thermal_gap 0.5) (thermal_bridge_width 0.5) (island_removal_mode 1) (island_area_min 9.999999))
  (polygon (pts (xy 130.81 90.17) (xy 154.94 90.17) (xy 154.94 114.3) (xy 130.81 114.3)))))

